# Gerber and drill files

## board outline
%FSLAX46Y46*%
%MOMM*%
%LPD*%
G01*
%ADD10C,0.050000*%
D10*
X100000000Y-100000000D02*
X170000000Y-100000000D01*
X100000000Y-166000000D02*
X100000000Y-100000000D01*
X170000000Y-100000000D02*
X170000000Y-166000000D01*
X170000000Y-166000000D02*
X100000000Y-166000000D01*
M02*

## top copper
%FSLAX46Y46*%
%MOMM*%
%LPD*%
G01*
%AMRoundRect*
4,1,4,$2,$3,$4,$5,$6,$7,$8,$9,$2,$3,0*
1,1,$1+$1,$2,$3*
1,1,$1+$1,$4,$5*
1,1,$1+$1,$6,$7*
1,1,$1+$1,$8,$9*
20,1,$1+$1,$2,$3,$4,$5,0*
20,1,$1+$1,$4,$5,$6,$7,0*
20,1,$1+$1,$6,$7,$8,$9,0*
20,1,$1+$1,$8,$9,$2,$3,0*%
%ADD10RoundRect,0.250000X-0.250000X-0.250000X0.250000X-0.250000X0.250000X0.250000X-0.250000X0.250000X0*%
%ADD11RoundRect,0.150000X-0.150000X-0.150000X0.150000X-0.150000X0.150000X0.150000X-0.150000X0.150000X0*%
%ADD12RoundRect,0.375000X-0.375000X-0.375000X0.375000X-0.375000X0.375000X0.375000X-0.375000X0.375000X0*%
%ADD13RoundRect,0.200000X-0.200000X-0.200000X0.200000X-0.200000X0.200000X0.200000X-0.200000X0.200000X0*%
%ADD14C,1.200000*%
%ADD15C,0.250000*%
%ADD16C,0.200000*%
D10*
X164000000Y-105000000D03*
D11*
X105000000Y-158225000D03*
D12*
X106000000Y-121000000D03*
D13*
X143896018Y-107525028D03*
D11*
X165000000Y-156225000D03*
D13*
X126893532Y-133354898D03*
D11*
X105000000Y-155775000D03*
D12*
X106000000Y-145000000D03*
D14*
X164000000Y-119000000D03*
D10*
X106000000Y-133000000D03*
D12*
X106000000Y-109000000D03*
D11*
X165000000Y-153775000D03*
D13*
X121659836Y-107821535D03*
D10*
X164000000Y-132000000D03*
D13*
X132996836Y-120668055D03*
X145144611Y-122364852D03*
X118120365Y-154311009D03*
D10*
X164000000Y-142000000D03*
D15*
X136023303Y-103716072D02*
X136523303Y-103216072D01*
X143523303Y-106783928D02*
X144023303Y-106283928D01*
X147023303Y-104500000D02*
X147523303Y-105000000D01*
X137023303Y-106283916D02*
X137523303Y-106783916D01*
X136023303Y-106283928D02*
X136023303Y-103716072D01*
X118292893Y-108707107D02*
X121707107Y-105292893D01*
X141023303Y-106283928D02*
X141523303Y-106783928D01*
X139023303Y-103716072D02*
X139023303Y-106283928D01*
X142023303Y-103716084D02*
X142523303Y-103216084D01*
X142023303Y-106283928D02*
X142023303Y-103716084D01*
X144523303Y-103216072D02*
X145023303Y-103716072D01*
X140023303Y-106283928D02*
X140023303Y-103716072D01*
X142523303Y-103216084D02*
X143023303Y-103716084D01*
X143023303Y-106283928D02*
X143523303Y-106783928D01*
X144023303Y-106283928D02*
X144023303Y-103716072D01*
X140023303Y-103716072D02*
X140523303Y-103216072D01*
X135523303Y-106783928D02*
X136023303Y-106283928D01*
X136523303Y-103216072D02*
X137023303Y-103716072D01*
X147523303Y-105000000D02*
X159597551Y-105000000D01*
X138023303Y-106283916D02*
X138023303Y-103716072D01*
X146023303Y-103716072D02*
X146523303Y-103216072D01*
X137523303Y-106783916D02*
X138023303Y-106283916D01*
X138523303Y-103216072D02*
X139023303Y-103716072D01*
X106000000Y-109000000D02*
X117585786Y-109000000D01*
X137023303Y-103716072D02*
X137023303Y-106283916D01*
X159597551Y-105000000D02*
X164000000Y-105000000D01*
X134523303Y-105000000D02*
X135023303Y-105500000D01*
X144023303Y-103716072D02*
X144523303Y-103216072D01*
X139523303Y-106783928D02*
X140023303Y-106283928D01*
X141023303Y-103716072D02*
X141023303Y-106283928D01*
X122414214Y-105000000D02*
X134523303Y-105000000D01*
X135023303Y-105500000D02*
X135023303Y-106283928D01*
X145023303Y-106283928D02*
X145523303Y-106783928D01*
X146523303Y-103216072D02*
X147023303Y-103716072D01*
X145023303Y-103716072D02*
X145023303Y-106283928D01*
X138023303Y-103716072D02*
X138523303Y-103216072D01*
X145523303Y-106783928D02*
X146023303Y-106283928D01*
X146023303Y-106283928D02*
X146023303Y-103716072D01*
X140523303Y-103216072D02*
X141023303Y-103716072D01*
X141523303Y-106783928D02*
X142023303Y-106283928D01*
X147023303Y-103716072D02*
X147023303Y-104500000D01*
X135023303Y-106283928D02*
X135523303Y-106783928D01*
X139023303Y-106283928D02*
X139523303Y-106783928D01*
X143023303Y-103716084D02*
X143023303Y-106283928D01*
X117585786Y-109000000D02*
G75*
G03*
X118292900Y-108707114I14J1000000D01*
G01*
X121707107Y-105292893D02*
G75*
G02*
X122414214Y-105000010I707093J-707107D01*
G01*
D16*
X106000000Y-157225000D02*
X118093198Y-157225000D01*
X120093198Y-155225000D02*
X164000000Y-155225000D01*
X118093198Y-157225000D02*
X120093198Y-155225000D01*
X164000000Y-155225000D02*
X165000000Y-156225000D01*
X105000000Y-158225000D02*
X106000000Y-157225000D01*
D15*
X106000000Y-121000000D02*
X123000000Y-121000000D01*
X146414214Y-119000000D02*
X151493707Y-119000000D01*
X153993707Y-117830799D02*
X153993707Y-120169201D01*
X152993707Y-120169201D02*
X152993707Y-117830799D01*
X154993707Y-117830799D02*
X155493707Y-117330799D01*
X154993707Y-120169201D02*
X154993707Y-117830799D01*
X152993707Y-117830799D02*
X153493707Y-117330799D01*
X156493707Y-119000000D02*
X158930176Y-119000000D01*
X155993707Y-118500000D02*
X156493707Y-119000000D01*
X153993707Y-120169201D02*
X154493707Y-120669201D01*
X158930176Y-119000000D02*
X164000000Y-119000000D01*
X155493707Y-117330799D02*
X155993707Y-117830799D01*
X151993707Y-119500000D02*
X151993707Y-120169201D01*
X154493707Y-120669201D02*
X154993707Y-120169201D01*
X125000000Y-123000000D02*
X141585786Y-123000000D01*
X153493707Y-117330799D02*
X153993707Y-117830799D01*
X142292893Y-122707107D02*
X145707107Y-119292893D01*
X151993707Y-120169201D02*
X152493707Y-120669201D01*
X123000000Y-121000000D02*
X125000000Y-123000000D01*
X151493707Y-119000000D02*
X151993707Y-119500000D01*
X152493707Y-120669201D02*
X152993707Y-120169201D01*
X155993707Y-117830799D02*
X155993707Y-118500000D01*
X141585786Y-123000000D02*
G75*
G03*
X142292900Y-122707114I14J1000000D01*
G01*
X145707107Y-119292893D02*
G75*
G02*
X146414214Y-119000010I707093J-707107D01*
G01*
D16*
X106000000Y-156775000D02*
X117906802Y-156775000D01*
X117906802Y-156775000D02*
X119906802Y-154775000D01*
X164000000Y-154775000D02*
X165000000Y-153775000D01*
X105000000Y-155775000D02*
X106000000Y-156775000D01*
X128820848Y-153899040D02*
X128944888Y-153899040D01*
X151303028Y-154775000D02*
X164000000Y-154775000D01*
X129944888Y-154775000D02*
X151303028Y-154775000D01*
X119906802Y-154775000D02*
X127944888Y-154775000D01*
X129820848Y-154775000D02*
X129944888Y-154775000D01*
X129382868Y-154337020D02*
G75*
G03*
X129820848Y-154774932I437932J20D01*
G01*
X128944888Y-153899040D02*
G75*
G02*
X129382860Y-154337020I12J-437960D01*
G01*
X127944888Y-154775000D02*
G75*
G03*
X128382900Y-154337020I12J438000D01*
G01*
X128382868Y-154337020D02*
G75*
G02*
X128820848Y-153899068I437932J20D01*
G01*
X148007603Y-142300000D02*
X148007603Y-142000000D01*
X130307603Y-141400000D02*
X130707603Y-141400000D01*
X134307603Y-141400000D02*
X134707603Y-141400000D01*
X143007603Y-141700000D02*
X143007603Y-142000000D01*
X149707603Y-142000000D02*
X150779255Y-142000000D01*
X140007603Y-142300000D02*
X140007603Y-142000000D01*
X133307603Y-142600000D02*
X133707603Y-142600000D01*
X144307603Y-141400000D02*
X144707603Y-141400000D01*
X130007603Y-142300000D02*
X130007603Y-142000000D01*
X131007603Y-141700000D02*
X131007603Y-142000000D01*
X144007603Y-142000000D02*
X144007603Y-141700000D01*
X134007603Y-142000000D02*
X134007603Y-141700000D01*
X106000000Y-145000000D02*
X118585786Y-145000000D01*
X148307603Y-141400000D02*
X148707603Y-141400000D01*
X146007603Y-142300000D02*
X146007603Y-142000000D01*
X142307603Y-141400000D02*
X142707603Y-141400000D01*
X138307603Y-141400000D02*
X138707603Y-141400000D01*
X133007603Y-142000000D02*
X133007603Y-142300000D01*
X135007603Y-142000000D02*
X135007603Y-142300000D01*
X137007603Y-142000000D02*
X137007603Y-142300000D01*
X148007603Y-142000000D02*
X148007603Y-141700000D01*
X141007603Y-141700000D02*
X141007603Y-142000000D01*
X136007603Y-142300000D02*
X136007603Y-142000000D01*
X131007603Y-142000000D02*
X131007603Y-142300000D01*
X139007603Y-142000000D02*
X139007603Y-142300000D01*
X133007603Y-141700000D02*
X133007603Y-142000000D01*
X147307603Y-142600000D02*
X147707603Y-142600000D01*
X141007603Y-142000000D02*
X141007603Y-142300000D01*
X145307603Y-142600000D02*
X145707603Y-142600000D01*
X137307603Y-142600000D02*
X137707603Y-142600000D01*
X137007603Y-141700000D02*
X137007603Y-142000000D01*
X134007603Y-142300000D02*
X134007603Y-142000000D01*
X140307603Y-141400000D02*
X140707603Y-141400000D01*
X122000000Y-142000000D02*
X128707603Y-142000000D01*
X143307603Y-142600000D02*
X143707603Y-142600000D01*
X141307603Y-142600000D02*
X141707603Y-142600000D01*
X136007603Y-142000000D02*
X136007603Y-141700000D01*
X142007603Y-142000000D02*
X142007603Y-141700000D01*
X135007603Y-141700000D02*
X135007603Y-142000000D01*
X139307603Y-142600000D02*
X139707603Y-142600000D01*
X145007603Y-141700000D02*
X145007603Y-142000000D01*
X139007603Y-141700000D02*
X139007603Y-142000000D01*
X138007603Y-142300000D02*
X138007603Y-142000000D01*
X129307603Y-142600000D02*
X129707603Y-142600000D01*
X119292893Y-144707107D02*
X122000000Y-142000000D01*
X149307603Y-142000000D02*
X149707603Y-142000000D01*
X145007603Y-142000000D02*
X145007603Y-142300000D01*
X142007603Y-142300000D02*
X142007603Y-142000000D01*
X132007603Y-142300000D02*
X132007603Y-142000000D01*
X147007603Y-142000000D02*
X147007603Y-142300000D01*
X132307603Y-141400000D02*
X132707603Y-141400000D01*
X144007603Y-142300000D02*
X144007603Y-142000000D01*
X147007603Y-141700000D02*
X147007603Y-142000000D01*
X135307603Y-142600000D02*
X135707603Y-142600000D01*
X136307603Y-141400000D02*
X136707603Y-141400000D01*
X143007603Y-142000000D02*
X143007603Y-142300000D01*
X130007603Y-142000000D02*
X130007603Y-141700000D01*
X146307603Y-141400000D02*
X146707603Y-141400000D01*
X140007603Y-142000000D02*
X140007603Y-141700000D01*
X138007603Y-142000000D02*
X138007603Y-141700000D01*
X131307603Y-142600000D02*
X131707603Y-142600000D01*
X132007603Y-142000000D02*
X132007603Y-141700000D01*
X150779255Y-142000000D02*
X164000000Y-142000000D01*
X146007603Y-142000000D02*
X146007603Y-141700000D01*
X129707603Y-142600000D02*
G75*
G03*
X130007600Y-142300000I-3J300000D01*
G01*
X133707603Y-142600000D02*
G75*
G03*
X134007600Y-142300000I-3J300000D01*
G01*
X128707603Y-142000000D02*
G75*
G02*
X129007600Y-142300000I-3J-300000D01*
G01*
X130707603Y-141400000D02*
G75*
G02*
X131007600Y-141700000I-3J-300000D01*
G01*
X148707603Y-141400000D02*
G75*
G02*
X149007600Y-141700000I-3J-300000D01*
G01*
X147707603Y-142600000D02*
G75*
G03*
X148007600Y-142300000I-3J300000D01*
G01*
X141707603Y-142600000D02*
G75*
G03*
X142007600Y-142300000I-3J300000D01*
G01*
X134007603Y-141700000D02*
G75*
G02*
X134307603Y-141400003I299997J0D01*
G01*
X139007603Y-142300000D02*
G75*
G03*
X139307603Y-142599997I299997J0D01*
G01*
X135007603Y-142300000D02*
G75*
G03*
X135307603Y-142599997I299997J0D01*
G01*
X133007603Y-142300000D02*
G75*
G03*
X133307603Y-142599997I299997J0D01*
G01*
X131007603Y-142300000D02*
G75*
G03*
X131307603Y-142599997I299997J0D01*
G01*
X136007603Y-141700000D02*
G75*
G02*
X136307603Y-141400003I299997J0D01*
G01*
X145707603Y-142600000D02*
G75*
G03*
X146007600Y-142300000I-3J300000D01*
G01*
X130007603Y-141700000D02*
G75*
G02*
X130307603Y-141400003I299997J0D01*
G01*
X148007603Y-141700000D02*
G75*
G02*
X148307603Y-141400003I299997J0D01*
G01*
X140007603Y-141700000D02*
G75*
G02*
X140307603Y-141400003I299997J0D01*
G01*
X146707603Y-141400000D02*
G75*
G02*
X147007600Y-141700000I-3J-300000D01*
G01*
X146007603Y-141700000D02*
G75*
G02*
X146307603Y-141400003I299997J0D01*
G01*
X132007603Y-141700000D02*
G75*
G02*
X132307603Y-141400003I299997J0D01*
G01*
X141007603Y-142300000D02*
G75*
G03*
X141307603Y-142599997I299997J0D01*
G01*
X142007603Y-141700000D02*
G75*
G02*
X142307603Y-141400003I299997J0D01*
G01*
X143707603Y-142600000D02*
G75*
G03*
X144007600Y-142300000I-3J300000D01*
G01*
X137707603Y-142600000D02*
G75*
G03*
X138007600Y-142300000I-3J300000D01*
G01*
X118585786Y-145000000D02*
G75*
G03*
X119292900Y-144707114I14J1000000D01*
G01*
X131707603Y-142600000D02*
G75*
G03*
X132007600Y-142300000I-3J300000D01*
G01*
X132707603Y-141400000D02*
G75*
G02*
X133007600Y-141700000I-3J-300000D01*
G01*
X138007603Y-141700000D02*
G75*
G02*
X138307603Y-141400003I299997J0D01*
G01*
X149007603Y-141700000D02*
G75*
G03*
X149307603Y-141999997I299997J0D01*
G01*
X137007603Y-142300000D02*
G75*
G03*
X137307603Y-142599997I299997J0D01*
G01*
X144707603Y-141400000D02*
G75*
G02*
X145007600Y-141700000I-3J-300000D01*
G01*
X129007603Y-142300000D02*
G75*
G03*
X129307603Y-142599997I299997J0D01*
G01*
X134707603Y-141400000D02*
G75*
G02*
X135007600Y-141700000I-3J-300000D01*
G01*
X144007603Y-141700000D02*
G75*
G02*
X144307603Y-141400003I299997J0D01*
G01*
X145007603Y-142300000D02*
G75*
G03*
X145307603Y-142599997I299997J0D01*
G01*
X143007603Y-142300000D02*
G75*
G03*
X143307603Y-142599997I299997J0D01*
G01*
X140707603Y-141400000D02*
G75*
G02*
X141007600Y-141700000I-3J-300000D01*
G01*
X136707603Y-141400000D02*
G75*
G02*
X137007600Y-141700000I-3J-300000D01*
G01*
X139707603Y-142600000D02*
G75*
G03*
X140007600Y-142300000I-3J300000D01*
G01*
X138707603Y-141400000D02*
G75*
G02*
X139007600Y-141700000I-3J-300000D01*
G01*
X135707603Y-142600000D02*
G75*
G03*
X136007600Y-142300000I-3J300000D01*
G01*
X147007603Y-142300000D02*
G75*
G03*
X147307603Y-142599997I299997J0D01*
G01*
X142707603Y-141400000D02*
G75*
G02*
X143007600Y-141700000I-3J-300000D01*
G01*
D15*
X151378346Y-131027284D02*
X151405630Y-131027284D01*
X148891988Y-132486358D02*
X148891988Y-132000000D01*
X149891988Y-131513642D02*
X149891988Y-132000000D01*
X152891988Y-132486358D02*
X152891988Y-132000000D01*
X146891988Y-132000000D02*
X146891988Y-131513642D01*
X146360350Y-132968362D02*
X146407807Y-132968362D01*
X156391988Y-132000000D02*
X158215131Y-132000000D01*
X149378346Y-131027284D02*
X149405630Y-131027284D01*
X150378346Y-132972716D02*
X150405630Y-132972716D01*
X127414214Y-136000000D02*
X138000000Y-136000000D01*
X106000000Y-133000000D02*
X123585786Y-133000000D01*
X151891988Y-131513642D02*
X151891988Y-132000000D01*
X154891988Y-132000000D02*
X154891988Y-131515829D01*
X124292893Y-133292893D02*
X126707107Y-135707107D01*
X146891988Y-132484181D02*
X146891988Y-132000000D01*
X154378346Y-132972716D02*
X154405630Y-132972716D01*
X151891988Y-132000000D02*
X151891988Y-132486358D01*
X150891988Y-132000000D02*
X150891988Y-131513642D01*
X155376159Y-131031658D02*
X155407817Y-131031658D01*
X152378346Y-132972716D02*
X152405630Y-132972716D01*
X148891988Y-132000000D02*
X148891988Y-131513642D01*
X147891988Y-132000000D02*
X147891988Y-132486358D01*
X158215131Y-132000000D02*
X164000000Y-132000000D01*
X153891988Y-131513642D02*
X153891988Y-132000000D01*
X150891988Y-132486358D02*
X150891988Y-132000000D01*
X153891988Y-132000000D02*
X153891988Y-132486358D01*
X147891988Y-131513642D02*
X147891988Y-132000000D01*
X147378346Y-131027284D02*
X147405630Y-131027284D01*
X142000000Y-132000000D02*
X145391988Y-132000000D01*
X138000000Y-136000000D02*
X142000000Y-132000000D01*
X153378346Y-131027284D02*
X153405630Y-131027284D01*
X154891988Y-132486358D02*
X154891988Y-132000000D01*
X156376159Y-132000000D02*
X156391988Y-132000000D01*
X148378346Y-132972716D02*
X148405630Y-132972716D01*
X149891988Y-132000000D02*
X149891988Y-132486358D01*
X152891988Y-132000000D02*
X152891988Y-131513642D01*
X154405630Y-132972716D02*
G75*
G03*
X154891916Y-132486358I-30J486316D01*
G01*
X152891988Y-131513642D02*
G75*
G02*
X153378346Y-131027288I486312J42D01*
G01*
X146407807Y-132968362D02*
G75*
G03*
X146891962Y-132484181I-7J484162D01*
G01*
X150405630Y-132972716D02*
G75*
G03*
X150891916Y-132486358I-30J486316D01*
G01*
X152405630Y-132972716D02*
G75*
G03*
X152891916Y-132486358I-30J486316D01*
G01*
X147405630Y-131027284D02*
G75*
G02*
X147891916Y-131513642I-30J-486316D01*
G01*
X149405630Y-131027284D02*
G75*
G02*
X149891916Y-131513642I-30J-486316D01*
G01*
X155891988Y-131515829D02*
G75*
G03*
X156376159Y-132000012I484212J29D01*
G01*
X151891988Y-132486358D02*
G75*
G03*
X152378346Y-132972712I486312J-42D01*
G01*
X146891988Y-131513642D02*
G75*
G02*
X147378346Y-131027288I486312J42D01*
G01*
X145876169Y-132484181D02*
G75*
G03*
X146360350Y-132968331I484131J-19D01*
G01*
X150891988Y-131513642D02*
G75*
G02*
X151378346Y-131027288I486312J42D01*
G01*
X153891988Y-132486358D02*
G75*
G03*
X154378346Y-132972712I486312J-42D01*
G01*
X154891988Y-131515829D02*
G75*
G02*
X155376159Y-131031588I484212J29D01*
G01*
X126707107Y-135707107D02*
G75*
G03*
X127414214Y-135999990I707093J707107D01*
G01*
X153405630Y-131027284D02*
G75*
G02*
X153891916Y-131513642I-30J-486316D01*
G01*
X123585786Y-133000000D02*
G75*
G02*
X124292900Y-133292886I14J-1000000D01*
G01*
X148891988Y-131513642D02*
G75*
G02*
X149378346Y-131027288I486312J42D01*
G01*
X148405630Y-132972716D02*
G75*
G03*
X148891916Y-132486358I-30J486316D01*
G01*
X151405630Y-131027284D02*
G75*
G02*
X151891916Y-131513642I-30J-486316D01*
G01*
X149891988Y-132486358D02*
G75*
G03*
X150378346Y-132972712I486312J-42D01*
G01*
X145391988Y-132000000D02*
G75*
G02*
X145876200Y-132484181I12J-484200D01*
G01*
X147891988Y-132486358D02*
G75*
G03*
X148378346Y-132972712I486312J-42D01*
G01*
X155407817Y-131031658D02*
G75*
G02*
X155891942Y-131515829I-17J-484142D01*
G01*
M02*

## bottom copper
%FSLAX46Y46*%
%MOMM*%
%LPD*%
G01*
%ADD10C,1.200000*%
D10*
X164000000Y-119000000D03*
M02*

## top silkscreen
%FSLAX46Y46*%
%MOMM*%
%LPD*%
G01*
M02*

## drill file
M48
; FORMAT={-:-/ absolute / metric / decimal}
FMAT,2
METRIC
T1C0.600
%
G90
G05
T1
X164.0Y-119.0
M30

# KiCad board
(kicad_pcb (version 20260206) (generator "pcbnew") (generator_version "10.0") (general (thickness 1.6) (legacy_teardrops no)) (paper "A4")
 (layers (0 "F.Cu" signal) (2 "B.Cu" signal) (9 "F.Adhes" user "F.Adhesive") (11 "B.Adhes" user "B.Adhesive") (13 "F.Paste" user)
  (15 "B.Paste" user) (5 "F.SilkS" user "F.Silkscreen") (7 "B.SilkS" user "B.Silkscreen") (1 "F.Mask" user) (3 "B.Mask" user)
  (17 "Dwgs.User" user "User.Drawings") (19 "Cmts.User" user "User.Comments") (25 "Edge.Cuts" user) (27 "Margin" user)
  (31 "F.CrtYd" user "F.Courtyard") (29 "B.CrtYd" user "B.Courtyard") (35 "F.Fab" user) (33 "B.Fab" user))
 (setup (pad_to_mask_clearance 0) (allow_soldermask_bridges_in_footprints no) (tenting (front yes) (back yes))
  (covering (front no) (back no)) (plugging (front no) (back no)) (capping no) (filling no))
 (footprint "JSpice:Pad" (layer "F.Cu") (at 164 105)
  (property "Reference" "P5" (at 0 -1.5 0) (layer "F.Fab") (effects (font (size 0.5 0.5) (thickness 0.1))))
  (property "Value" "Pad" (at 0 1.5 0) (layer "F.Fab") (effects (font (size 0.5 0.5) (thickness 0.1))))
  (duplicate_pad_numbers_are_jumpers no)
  (pad "1" smd roundrect (at 0 0) (size 1 1) (layers "F.Cu" "F.Mask") (roundrect_rratio 0.25) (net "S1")))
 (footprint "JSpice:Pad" (layer "F.Cu") (at 105 158.225)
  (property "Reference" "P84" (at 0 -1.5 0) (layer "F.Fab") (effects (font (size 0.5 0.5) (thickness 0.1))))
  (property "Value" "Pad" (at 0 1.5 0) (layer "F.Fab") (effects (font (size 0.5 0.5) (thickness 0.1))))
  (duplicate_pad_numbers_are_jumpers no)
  (pad "1" smd roundrect (at 0 0) (size 0.6 0.6) (layers "F.Cu" "F.Mask") (roundrect_rratio 0.25) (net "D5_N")))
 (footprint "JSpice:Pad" (layer "F.Cu") (at 106 121)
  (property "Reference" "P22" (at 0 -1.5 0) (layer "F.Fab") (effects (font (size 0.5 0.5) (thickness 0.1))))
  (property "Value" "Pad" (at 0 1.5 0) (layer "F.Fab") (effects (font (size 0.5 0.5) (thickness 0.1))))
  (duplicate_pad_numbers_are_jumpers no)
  (pad "1" smd roundrect (at 0 0) (size 1.5 1.5) (layers "F.Cu" "F.Mask") (roundrect_rratio 0.25) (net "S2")))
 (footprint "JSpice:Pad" (layer "F.Cu") (at 143.896018 107.525028)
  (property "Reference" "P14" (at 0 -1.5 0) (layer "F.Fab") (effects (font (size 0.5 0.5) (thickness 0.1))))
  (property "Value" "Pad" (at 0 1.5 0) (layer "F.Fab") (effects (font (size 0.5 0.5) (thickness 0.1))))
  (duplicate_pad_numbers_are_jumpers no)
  (pad "1" smd roundrect (at 0 0) (size 0.8 0.8) (layers "F.Cu" "F.Mask") (roundrect_rratio 0.25) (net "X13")))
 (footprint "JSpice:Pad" (layer "F.Cu") (at 165 156.225)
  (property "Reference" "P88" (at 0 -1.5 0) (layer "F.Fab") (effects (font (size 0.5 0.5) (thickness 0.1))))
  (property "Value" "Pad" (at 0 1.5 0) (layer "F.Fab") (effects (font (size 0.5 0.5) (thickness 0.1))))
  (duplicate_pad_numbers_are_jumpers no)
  (pad "1" smd roundrect (at 0 0) (size 0.6 0.6) (layers "F.Cu" "F.Mask") (roundrect_rratio 0.25) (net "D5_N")))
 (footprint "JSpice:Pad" (layer "F.Cu") (at 126.893532 133.354898)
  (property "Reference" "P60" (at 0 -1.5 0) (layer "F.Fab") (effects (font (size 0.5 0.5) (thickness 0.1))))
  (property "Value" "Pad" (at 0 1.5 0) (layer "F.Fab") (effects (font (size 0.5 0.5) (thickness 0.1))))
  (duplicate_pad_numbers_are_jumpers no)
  (pad "1" smd roundrect (at 0 0) (size 0.8 0.8) (layers "F.Cu" "F.Mask") (roundrect_rratio 0.25) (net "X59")))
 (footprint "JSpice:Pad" (layer "F.Cu") (at 105 155.775)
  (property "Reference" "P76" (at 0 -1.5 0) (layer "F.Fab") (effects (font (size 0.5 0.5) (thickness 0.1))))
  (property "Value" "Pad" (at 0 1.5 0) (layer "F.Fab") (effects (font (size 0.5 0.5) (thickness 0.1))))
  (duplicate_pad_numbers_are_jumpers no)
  (pad "1" smd roundrect (at 0 0) (size 0.6 0.6) (layers "F.Cu" "F.Mask") (roundrect_rratio 0.25) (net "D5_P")))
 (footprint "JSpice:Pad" (layer "F.Cu") (at 106 145)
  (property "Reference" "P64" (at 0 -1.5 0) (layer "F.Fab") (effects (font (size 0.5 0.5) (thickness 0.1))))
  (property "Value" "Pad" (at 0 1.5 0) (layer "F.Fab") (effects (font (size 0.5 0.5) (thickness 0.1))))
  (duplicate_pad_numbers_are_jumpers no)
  (pad "1" smd roundrect (at 0 0) (size 1.5 1.5) (layers "F.Cu" "F.Mask") (roundrect_rratio 0.25) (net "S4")))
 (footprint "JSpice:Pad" (layer "F.Cu") (at 164 119)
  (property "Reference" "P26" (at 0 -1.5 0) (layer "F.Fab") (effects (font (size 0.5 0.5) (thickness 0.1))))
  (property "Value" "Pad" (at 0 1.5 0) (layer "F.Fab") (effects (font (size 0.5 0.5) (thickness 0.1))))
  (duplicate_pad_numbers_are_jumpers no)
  (pad "1" thru_hole circle (at 0 0) (size 1.2 1.2) (drill 0.6) (layers "*.Cu" "*.Mask") (remove_unused_layers no) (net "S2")))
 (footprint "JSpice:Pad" (layer "F.Cu") (at 106 133)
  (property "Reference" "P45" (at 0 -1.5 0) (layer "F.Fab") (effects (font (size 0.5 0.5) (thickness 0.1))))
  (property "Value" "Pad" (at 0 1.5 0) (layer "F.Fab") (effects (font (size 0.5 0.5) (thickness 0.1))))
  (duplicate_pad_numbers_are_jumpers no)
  (pad "1" smd roundrect (at 0 0) (size 1 1) (layers "F.Cu" "F.Mask") (roundrect_rratio 0.25) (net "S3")))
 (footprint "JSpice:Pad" (layer "F.Cu") (at 106 109)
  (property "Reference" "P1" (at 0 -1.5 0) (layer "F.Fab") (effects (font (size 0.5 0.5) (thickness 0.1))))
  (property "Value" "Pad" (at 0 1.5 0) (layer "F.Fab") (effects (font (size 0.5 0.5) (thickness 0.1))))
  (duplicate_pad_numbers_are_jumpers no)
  (pad "1" smd roundrect (at 0 0) (size 1.5 1.5) (layers "F.Cu" "F.Mask") (roundrect_rratio 0.25) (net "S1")))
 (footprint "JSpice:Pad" (layer "F.Cu") (at 165 153.775)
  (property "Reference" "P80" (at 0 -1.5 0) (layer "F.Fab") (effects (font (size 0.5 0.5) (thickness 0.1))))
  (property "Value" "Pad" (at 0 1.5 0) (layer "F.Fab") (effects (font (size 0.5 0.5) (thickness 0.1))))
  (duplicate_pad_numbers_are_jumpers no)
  (pad "1" smd roundrect (at 0 0) (size 0.6 0.6) (layers "F.Cu" "F.Mask") (roundrect_rratio 0.25) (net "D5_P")))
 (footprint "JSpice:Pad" (layer "F.Cu") (at 121.659836 107.821535)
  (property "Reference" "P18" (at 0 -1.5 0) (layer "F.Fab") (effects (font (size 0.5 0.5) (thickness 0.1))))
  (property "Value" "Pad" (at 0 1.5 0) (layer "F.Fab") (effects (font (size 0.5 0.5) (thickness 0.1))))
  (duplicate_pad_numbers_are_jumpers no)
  (pad "1" smd roundrect (at 0 0) (size 0.8 0.8) (layers "F.Cu" "F.Mask") (roundrect_rratio 0.25) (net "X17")))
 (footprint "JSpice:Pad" (layer "F.Cu") (at 164 132)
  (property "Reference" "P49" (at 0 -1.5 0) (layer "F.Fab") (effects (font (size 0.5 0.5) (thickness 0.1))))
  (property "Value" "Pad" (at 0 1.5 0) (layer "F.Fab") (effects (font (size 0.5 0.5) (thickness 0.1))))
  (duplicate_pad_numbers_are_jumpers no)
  (pad "1" smd roundrect (at 0 0) (size 1 1) (layers "F.Cu" "F.Mask") (roundrect_rratio 0.25) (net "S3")))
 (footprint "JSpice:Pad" (layer "F.Cu") (at 132.996836 120.668055)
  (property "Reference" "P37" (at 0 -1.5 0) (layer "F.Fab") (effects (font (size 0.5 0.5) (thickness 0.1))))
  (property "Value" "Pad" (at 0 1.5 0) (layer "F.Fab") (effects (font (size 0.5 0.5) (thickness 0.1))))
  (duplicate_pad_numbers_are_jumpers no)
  (pad "1" smd roundrect (at 0 0) (size 0.8 0.8) (layers "F.Cu" "F.Mask") (roundrect_rratio 0.25) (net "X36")))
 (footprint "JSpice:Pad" (layer "F.Cu") (at 145.144611 122.364852)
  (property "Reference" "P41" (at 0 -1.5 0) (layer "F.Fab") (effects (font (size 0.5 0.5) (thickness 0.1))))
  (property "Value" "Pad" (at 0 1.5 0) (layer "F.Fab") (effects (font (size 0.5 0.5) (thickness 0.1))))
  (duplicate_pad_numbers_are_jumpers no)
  (pad "1" smd roundrect (at 0 0) (size 0.8 0.8) (layers "F.Cu" "F.Mask") (roundrect_rratio 0.25) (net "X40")))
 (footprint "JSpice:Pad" (layer "F.Cu") (at 118.120365 154.311009)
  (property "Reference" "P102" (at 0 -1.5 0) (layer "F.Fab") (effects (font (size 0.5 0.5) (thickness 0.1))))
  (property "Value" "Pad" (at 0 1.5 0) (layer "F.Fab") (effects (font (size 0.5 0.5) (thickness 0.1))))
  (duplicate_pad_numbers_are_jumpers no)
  (pad "1" smd roundrect (at 0 0) (size 0.8 0.8) (layers "F.Cu" "F.Mask") (roundrect_rratio 0.25) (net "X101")))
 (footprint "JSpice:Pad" (layer "F.Cu") (at 164 142)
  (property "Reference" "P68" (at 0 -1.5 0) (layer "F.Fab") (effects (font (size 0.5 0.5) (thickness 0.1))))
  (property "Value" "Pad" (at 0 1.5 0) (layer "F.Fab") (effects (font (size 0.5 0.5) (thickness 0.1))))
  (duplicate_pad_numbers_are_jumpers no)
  (pad "1" smd roundrect (at 0 0) (size 1 1) (layers "F.Cu" "F.Mask") (roundrect_rratio 0.25) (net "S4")))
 (gr_line (start 100 100) (end 170 100) (stroke (width 0.05) (type default)) (layer "Edge.Cuts"))
 (gr_line (start 100 166) (end 100 100) (stroke (width 0.05) (type default)) (layer "Edge.Cuts"))
 (gr_line (start 170 100) (end 170 166) (stroke (width 0.05) (type default)) (layer "Edge.Cuts"))
 (gr_line (start 170 166) (end 100 166) (stroke (width 0.05) (type default)) (layer "Edge.Cuts"))
 (segment (start 136.023303 103.716072) (end 136.523303 103.216072) (width 0.25) (layer "F.Cu") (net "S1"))
 (segment (start 143.523303 106.783928) (end 144.023303 106.283928) (width 0.25) (layer "F.Cu") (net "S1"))
 (segment (start 147.023303 104.5) (end 147.523303 105) (width 0.25) (layer "F.Cu") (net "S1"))
 (segment (start 137.023303 106.283916) (end 137.523303 106.783916) (width 0.25) (layer "F.Cu") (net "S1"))
 (segment (start 136.023303 106.283928) (end 136.023303 103.716072) (width 0.25) (layer "F.Cu") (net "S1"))
 (segment (start 118.292893 108.707107) (end 121.707107 105.292893) (width 0.25) (layer "F.Cu") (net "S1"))
 (segment (start 141.023303 106.283928) (end 141.523303 106.783928) (width 0.25) (layer "F.Cu") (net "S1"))
 (segment (start 139.023303 103.716072) (end 139.023303 106.283928) (width 0.25) (layer "F.Cu") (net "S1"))
 (segment (start 142.023303 103.716084) (end 142.523303 103.216084) (width 0.25) (layer "F.Cu") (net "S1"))
 (segment (start 142.023303 106.283928) (end 142.023303 103.716084) (width 0.25) (layer "F.Cu") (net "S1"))
 (segment (start 144.523303 103.216072) (end 145.023303 103.716072) (width 0.25) (layer "F.Cu") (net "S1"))
 (segment (start 140.023303 106.283928) (end 140.023303 103.716072) (width 0.25) (layer "F.Cu") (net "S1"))
 (segment (start 142.523303 103.216084) (end 143.023303 103.716084) (width 0.25) (layer "F.Cu") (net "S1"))
 (segment (start 143.023303 106.283928) (end 143.523303 106.783928) (width 0.25) (layer "F.Cu") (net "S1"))
 (segment (start 144.023303 106.283928) (end 144.023303 103.716072) (width 0.25) (layer "F.Cu") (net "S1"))
 (segment (start 140.023303 103.716072) (end 140.523303 103.216072) (width 0.25) (layer "F.Cu") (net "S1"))
 (segment (start 135.523303 106.783928) (end 136.023303 106.283928) (width 0.25) (layer "F.Cu") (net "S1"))
 (segment (start 136.523303 103.216072) (end 137.023303 103.716072) (width 0.25) (layer "F.Cu") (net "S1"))
 (segment (start 147.523303 105) (end 159.597551 105) (width 0.25) (layer "F.Cu") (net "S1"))
 (segment (start 138.023303 106.283916) (end 138.023303 103.716072) (width 0.25) (layer "F.Cu") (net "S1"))
 (segment (start 146.023303 103.716072) (end 146.523303 103.216072) (width 0.25) (layer "F.Cu") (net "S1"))
 (segment (start 137.523303 106.783916) (end 138.023303 106.283916) (width 0.25) (layer "F.Cu") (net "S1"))
 (segment (start 138.523303 103.216072) (end 139.023303 103.716072) (width 0.25) (layer "F.Cu") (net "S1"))
 (segment (start 106 109) (end 117.585786 109) (width 0.25) (layer "F.Cu") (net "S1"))
 (segment (start 137.023303 103.716072) (end 137.023303 106.283916) (width 0.25) (layer "F.Cu") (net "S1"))
 (segment (start 159.597551 105) (end 164 105) (width 0.25) (layer "F.Cu") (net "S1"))
 (segment (start 134.523303 105) (end 135.023303 105.5) (width 0.25) (layer "F.Cu") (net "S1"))
 (segment (start 144.023303 103.716072) (end 144.523303 103.216072) (width 0.25) (layer "F.Cu") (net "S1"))
 (segment (start 139.523303 106.783928) (end 140.023303 106.283928) (width 0.25) (layer "F.Cu") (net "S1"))
 (segment (start 141.023303 103.716072) (end 141.023303 106.283928) (width 0.25) (layer "F.Cu") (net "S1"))
 (segment (start 122.414214 105) (end 134.523303 105) (width 0.25) (layer "F.Cu") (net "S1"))
 (segment (start 135.023303 105.5) (end 135.023303 106.283928) (width 0.25) (layer "F.Cu") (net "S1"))
 (segment (start 145.023303 106.283928) (end 145.523303 106.783928) (width 0.25) (layer "F.Cu") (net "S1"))
 (segment (start 146.523303 103.216072) (end 147.023303 103.716072) (width 0.25) (layer "F.Cu") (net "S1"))
 (segment (start 145.023303 103.716072) (end 145.023303 106.283928) (width 0.25) (layer "F.Cu") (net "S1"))
 (segment (start 138.023303 103.716072) (end 138.523303 103.216072) (width 0.25) (layer "F.Cu") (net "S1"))
 (segment (start 145.523303 106.783928) (end 146.023303 106.283928) (width 0.25) (layer "F.Cu") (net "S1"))
 (segment (start 146.023303 106.283928) (end 146.023303 103.716072) (width 0.25) (layer "F.Cu") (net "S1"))
 (segment (start 140.523303 103.216072) (end 141.023303 103.716072) (width 0.25) (layer "F.Cu") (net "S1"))
 (segment (start 141.523303 106.783928) (end 142.023303 106.283928) (width 0.25) (layer "F.Cu") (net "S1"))
 (segment (start 147.023303 103.716072) (end 147.023303 104.5) (width 0.25) (layer "F.Cu") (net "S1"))
 (segment (start 135.023303 106.283928) (end 135.523303 106.783928) (width 0.25) (layer "F.Cu") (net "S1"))
 (segment (start 139.023303 106.283928) (end 139.523303 106.783928) (width 0.25) (layer "F.Cu") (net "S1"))
 (segment (start 143.023303 103.716084) (end 143.023303 106.283928) (width 0.25) (layer "F.Cu") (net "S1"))
 (arc (start 117.585786 109) (mid 117.96847 108.92388) (end 118.292893 108.707107) (width 0.25) (layer "F.Cu") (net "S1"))
 (arc (start 121.707107 105.292893) (mid 122.03153 105.07612) (end 122.414214 105) (width 0.25) (layer "F.Cu") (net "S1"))
 (segment (start 106 157.225) (end 118.093198 157.225) (width 0.2) (layer "F.Cu") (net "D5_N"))
 (segment (start 120.093198 155.225) (end 164 155.225) (width 0.2) (layer "F.Cu") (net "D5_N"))
 (segment (start 118.093198 157.225) (end 120.093198 155.225) (width 0.2) (layer "F.Cu") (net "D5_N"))
 (segment (start 164 155.225) (end 165 156.225) (width 0.2) (layer "F.Cu") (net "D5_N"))
 (segment (start 105 158.225) (end 106 157.225) (width 0.2) (layer "F.Cu") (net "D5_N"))
 (segment (start 106 121) (end 123 121) (width 0.25) (layer "F.Cu") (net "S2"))
 (segment (start 146.414214 119) (end 151.493707 119) (width 0.25) (layer "F.Cu") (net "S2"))
 (segment (start 153.993707 117.830799) (end 153.993707 120.169201) (width 0.25) (layer "F.Cu") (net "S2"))
 (segment (start 152.993707 120.169201) (end 152.993707 117.830799) (width 0.25) (layer "F.Cu") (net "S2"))
 (segment (start 154.993707 117.830799) (end 155.493707 117.330799) (width 0.25) (layer "F.Cu") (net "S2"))
 (segment (start 154.993707 120.169201) (end 154.993707 117.830799) (width 0.25) (layer "F.Cu") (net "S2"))
 (segment (start 152.993707 117.830799) (end 153.493707 117.330799) (width 0.25) (layer "F.Cu") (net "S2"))
 (segment (start 156.493707 119) (end 158.930176 119) (width 0.25) (layer "F.Cu") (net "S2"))
 (segment (start 155.993707 118.5) (end 156.493707 119) (width 0.25) (layer "F.Cu") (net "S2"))
 (segment (start 153.993707 120.169201) (end 154.493707 120.669201) (width 0.25) (layer "F.Cu") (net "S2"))
 (segment (start 158.930176 119) (end 164 119) (width 0.25) (layer "F.Cu") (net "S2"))
 (segment (start 155.493707 117.330799) (end 155.993707 117.830799) (width 0.25) (layer "F.Cu") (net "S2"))
 (segment (start 151.993707 119.5) (end 151.993707 120.169201) (width 0.25) (layer "F.Cu") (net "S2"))
 (segment (start 154.493707 120.669201) (end 154.993707 120.169201) (width 0.25) (layer "F.Cu") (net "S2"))
 (segment (start 125 123) (end 141.585786 123) (width 0.25) (layer "F.Cu") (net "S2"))
 (segment (start 153.493707 117.330799) (end 153.993707 117.830799) (width 0.25) (layer "F.Cu") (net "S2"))
 (segment (start 142.292893 122.707107) (end 145.707107 119.292893) (width 0.25) (layer "F.Cu") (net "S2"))
 (segment (start 151.993707 120.169201) (end 152.493707 120.669201) (width 0.25) (layer "F.Cu") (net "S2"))
 (segment (start 123 121) (end 125 123) (width 0.25) (layer "F.Cu") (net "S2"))
 (segment (start 151.493707 119) (end 151.993707 119.5) (width 0.25) (layer "F.Cu") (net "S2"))
 (segment (start 152.493707 120.669201) (end 152.993707 120.169201) (width 0.25) (layer "F.Cu") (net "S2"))
 (segment (start 155.993707 117.830799) (end 155.993707 118.5) (width 0.25) (layer "F.Cu") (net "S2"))
 (arc (start 141.585786 123) (mid 141.96847 122.92388) (end 142.292893 122.707107) (width 0.25) (layer "F.Cu") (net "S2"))
 (arc (start 145.707107 119.292893) (mid 146.03153 119.07612) (end 146.414214 119) (width 0.25) (layer "F.Cu") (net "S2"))
 (segment (start 106 156.775) (end 117.906802 156.775) (width 0.2) (layer "F.Cu") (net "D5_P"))
 (segment (start 117.906802 156.775) (end 119.906802 154.775) (width 0.2) (layer "F.Cu") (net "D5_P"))
 (segment (start 164 154.775) (end 165 153.775) (width 0.2) (layer "F.Cu") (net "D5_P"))
 (segment (start 105 155.775) (end 106 156.775) (width 0.2) (layer "F.Cu") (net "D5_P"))
 (segment (start 128.820848 153.89904) (end 128.944888 153.89904) (width 0.2) (layer "F.Cu") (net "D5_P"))
 (segment (start 151.303028 154.775) (end 164 154.775) (width 0.2) (layer "F.Cu") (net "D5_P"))
 (segment (start 129.944888 154.775) (end 151.303028 154.775) (width 0.2) (layer "F.Cu") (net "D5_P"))
 (segment (start 119.906802 154.775) (end 127.944888 154.775) (width 0.2) (layer "F.Cu") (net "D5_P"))
 (segment (start 129.820848 154.775) (end 129.944888 154.775) (width 0.2) (layer "F.Cu") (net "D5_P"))
 (arc (start 129.382868 154.33702) (mid 129.511149 154.646719) (end 129.820848 154.775) (width 0.2) (layer "F.Cu") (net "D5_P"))
 (arc (start 128.944888 153.89904) (mid 129.254587 154.027321) (end 129.382868 154.33702) (width 0.2) (layer "F.Cu") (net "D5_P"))
 (arc (start 127.944888 154.775) (mid 128.254587 154.646719) (end 128.382868 154.33702) (width 0.2) (layer "F.Cu") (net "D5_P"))
 (arc (start 128.382868 154.33702) (mid 128.511149 154.027321) (end 128.820848 153.89904) (width 0.2) (layer "F.Cu") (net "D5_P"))
 (segment (start 148.007603 142.3) (end 148.007603 142) (width 0.2) (layer "F.Cu") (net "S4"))
 (segment (start 130.307603 141.4) (end 130.707603 141.4) (width 0.2) (layer "F.Cu") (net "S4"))
 (segment (start 134.307603 141.4) (end 134.707603 141.4) (width 0.2) (layer "F.Cu") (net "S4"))
 (segment (start 143.007603 141.7) (end 143.007603 142) (width 0.2) (layer "F.Cu") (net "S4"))
 (segment (start 149.707603 142) (end 150.779255 142) (width 0.2) (layer "F.Cu") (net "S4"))
 (segment (start 140.007603 142.3) (end 140.007603 142) (width 0.2) (layer "F.Cu") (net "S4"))
 (segment (start 133.307603 142.6) (end 133.707603 142.6) (width 0.2) (layer "F.Cu") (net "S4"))
 (segment (start 144.307603 141.4) (end 144.707603 141.4) (width 0.2) (layer "F.Cu") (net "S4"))
 (segment (start 130.007603 142.3) (end 130.007603 142) (width 0.2) (layer "F.Cu") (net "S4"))
 (segment (start 131.007603 141.7) (end 131.007603 142) (width 0.2) (layer "F.Cu") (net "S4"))
 (segment (start 144.007603 142) (end 144.007603 141.7) (width 0.2) (layer "F.Cu") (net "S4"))
 (segment (start 134.007603 142) (end 134.007603 141.7) (width 0.2) (layer "F.Cu") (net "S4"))
 (segment (start 106 145) (end 118.585786 145) (width 0.2) (layer "F.Cu") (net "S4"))
 (segment (start 148.307603 141.4) (end 148.707603 141.4) (width 0.2) (layer "F.Cu") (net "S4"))
 (segment (start 146.007603 142.3) (end 146.007603 142) (width 0.2) (layer "F.Cu") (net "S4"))
 (segment (start 142.307603 141.4) (end 142.707603 141.4) (width 0.2) (layer "F.Cu") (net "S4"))
 (segment (start 138.307603 141.4) (end 138.707603 141.4) (width 0.2) (layer "F.Cu") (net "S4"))
 (segment (start 133.007603 142) (end 133.007603 142.3) (width 0.2) (layer "F.Cu") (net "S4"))
 (segment (start 135.007603 142) (end 135.007603 142.3) (width 0.2) (layer "F.Cu") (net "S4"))
 (segment (start 137.007603 142) (end 137.007603 142.3) (width 0.2) (layer "F.Cu") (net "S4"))
 (segment (start 148.007603 142) (end 148.007603 141.7) (width 0.2) (layer "F.Cu") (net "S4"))
 (segment (start 141.007603 141.7) (end 141.007603 142) (width 0.2) (layer "F.Cu") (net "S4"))
 (segment (start 136.007603 142.3) (end 136.007603 142) (width 0.2) (layer "F.Cu") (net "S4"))
 (segment (start 131.007603 142) (end 131.007603 142.3) (width 0.2) (layer "F.Cu") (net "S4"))
 (segment (start 139.007603 142) (end 139.007603 142.3) (width 0.2) (layer "F.Cu") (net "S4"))
 (segment (start 133.007603 141.7) (end 133.007603 142) (width 0.2) (layer "F.Cu") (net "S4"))
 (segment (start 147.307603 142.6) (end 147.707603 142.6) (width 0.2) (layer "F.Cu") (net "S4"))
 (segment (start 141.007603 142) (end 141.007603 142.3) (width 0.2) (layer "F.Cu") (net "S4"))
 (segment (start 145.307603 142.6) (end 145.707603 142.6) (width 0.2) (layer "F.Cu") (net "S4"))
 (segment (start 137.307603 142.6) (end 137.707603 142.6) (width 0.2) (layer "F.Cu") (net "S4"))
 (segment (start 137.007603 141.7) (end 137.007603 142) (width 0.2) (layer "F.Cu") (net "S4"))
 (segment (start 134.007603 142.3) (end 134.007603 142) (width 0.2) (layer "F.Cu") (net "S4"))
 (segment (start 140.307603 141.4) (end 140.707603 141.4) (width 0.2) (layer "F.Cu") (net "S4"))
 (segment (start 122 142) (end 128.707603 142) (width 0.2) (layer "F.Cu") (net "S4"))
 (segment (start 143.307603 142.6) (end 143.707603 142.6) (width 0.2) (layer "F.Cu") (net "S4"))
 (segment (start 141.307603 142.6) (end 141.707603 142.6) (width 0.2) (layer "F.Cu") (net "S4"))
 (segment (start 136.007603 142) (end 136.007603 141.7) (width 0.2) (layer "F.Cu") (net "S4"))
 (segment (start 142.007603 142) (end 142.007603 141.7) (width 0.2) (layer "F.Cu") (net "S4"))
 (segment (start 135.007603 141.7) (end 135.007603 142) (width 0.2) (layer "F.Cu") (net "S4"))
 (segment (start 139.307603 142.6) (end 139.707603 142.6) (width 0.2) (layer "F.Cu") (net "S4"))
 (segment (start 145.007603 141.7) (end 145.007603 142) (width 0.2) (layer "F.Cu") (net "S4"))
 (segment (start 139.007603 141.7) (end 139.007603 142) (width 0.2) (layer "F.Cu") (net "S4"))
 (segment (start 138.007603 142.3) (end 138.007603 142) (width 0.2) (layer "F.Cu") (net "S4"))
 (segment (start 129.307603 142.6) (end 129.707603 142.6) (width 0.2) (layer "F.Cu") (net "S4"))
 (segment (start 119.292893 144.707107) (end 122 142) (width 0.2) (layer "F.Cu") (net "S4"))
 (segment (start 149.307603 142) (end 149.707603 142) (width 0.2) (layer "F.Cu") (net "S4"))
 (segment (start 145.007603 142) (end 145.007603 142.3) (width 0.2) (layer "F.Cu") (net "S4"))
 (segment (start 142.007603 142.3) (end 142.007603 142) (width 0.2) (layer "F.Cu") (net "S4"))
 (segment (start 132.007603 142.3) (end 132.007603 142) (width 0.2) (layer "F.Cu") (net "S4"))
 (segment (start 147.007603 142) (end 147.007603 142.3) (width 0.2) (layer "F.Cu") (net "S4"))
 (segment (start 132.307603 141.4) (end 132.707603 141.4) (width 0.2) (layer "F.Cu") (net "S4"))
 (segment (start 144.007603 142.3) (end 144.007603 142) (width 0.2) (layer "F.Cu") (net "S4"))
 (segment (start 147.007603 141.7) (end 147.007603 142) (width 0.2) (layer "F.Cu") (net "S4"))
 (segment (start 135.307603 142.6) (end 135.707603 142.6) (width 0.2) (layer "F.Cu") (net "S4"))
 (segment (start 136.307603 141.4) (end 136.707603 141.4) (width 0.2) (layer "F.Cu") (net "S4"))
 (segment (start 143.007603 142) (end 143.007603 142.3) (width 0.2) (layer "F.Cu") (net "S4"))
 (segment (start 130.007603 142) (end 130.007603 141.7) (width 0.2) (layer "F.Cu") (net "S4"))
 (segment (start 146.307603 141.4) (end 146.707603 141.4) (width 0.2) (layer "F.Cu") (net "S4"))
 (segment (start 140.007603 142) (end 140.007603 141.7) (width 0.2) (layer "F.Cu") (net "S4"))
 (segment (start 138.007603 142) (end 138.007603 141.7) (width 0.2) (layer "F.Cu") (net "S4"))
 (segment (start 131.307603 142.6) (end 131.707603 142.6) (width 0.2) (layer "F.Cu") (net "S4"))
 (segment (start 132.007603 142) (end 132.007603 141.7) (width 0.2) (layer "F.Cu") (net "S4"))
 (segment (start 150.779255 142) (end 164 142) (width 0.2) (layer "F.Cu") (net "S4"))
 (segment (start 146.007603 142) (end 146.007603 141.7) (width 0.2) (layer "F.Cu") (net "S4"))
 (arc (start 129.707603 142.6) (mid 129.919735 142.512132) (end 130.007603 142.3) (width 0.2) (layer "F.Cu") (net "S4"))
 (arc (start 133.707603 142.6) (mid 133.919735 142.512132) (end 134.007603 142.3) (width 0.2) (layer "F.Cu") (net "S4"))
 (arc (start 128.707603 142) (mid 128.919735 142.087868) (end 129.007603 142.3) (width 0.2) (layer "F.Cu") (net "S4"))
 (arc (start 130.707603 141.4) (mid 130.919735 141.487868) (end 131.007603 141.7) (width 0.2) (layer "F.Cu") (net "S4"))
 (arc (start 148.707603 141.4) (mid 148.919735 141.487868) (end 149.007603 141.7) (width 0.2) (layer "F.Cu") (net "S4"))
 (arc (start 147.707603 142.6) (mid 147.919735 142.512132) (end 148.007603 142.3) (width 0.2) (layer "F.Cu") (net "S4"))
 (arc (start 141.707603 142.6) (mid 141.919735 142.512132) (end 142.007603 142.3) (width 0.2) (layer "F.Cu") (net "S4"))
 (arc (start 134.007603 141.7) (mid 134.095471 141.487868) (end 134.307603 141.4) (width 0.2) (layer "F.Cu") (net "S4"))
 (arc (start 139.007603 142.3) (mid 139.095471 142.512132) (end 139.307603 142.6) (width 0.2) (layer "F.Cu") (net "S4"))
 (arc (start 135.007603 142.3) (mid 135.095471 142.512132) (end 135.307603 142.6) (width 0.2) (layer "F.Cu") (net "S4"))
 (arc (start 133.007603 142.3) (mid 133.095471 142.512132) (end 133.307603 142.6) (width 0.2) (layer "F.Cu") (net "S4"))
 (arc (start 131.007603 142.3) (mid 131.095471 142.512132) (end 131.307603 142.6) (width 0.2) (layer "F.Cu") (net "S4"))
 (arc (start 136.007603 141.7) (mid 136.095471 141.487868) (end 136.307603 141.4) (width 0.2) (layer "F.Cu") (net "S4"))
 (arc (start 145.707603 142.6) (mid 145.919735 142.512132) (end 146.007603 142.3) (width 0.2) (layer "F.Cu") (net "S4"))
 (arc (start 130.007603 141.7) (mid 130.095471 141.487868) (end 130.307603 141.4) (width 0.2) (layer "F.Cu") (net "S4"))
 (arc (start 148.007603 141.7) (mid 148.095471 141.487868) (end 148.307603 141.4) (width 0.2) (layer "F.Cu") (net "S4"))
 (arc (start 140.007603 141.7) (mid 140.095471 141.487868) (end 140.307603 141.4) (width 0.2) (layer "F.Cu") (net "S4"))
 (arc (start 146.707603 141.4) (mid 146.919735 141.487868) (end 147.007603 141.7) (width 0.2) (layer "F.Cu") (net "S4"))
 (arc (start 146.007603 141.7) (mid 146.095471 141.487868) (end 146.307603 141.4) (width 0.2) (layer "F.Cu") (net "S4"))
 (arc (start 132.007603 141.7) (mid 132.095471 141.487868) (end 132.307603 141.4) (width 0.2) (layer "F.Cu") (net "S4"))
 (arc (start 141.007603 142.3) (mid 141.095471 142.512132) (end 141.307603 142.6) (width 0.2) (layer "F.Cu") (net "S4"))
 (arc (start 142.007603 141.7) (mid 142.095471 141.487868) (end 142.307603 141.4) (width 0.2) (layer "F.Cu") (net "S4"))
 (arc (start 143.707603 142.6) (mid 143.919735 142.512132) (end 144.007603 142.3) (width 0.2) (layer "F.Cu") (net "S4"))
 (arc (start 137.707603 142.6) (mid 137.919735 142.512132) (end 138.007603 142.3) (width 0.2) (layer "F.Cu") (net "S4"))
 (arc (start 118.585786 145) (mid 118.96847 144.92388) (end 119.292893 144.707107) (width 0.2) (layer "F.Cu") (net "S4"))
 (arc (start 131.707603 142.6) (mid 131.919735 142.512132) (end 132.007603 142.3) (width 0.2) (layer "F.Cu") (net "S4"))
 (arc (start 132.707603 141.4) (mid 132.919735 141.487868) (end 133.007603 141.7) (width 0.2) (layer "F.Cu") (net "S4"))
 (arc (start 138.007603 141.7) (mid 138.095471 141.487868) (end 138.307603 141.4) (width 0.2) (layer "F.Cu") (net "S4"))
 (arc (start 149.007603 141.7) (mid 149.095471 141.912132) (end 149.307603 142) (width 0.2) (layer "F.Cu") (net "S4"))
 (arc (start 137.007603 142.3) (mid 137.095471 142.512132) (end 137.307603 142.6) (width 0.2) (layer "F.Cu") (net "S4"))
 (arc (start 144.707603 141.4) (mid 144.919735 141.487868) (end 145.007603 141.7) (width 0.2) (layer "F.Cu") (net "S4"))
 (arc (start 129.007603 142.3) (mid 129.095471 142.512132) (end 129.307603 142.6) (width 0.2) (layer "F.Cu") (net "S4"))
 (arc (start 134.707603 141.4) (mid 134.919735 141.487868) (end 135.007603 141.7) (width 0.2) (layer "F.Cu") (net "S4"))
 (arc (start 144.007603 141.7) (mid 144.095471 141.487868) (end 144.307603 141.4) (width 0.2) (layer "F.Cu") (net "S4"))
 (arc (start 145.007603 142.3) (mid 145.095471 142.512132) (end 145.307603 142.6) (width 0.2) (layer "F.Cu") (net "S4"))
 (arc (start 143.007603 142.3) (mid 143.095471 142.512132) (end 143.307603 142.6) (width 0.2) (layer "F.Cu") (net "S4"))
 (arc (start 140.707603 141.4) (mid 140.919735 141.487868) (end 141.007603 141.7) (width 0.2) (layer "F.Cu") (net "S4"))
 (arc (start 136.707603 141.4) (mid 136.919735 141.487868) (end 137.007603 141.7) (width 0.2) (layer "F.Cu") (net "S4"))
 (arc (start 139.707603 142.6) (mid 139.919735 142.512132) (end 140.007603 142.3) (width 0.2) (layer "F.Cu") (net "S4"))
 (arc (start 138.707603 141.4) (mid 138.919735 141.487868) (end 139.007603 141.7) (width 0.2) (layer "F.Cu") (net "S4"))
 (arc (start 135.707603 142.6) (mid 135.919735 142.512132) (end 136.007603 142.3) (width 0.2) (layer "F.Cu") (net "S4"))
 (arc (start 147.007603 142.3) (mid 147.095471 142.512132) (end 147.307603 142.6) (width 0.2) (layer "F.Cu") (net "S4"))
 (arc (start 142.707603 141.4) (mid 142.919735 141.487868) (end 143.007603 141.7) (width 0.2) (layer "F.Cu") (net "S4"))
 (segment (start 151.378346 131.027284) (end 151.40563 131.027284) (width 0.25) (layer "F.Cu") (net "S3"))
 (segment (start 148.891988 132.486358) (end 148.891988 132) (width 0.25) (layer "F.Cu") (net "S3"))
 (segment (start 149.891988 131.513642) (end 149.891988 132) (width 0.25) (layer "F.Cu") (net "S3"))
 (segment (start 152.891988 132.486358) (end 152.891988 132) (width 0.25) (layer "F.Cu") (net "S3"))
 (segment (start 146.891988 132) (end 146.891988 131.513642) (width 0.25) (layer "F.Cu") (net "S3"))
 (segment (start 146.36035 132.968362) (end 146.407807 132.968362) (width 0.25) (layer "F.Cu") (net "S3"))
 (segment (start 156.391988 132) (end 158.215131 132) (width 0.25) (layer "F.Cu") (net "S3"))
 (segment (start 149.378346 131.027284) (end 149.40563 131.027284) (width 0.25) (layer "F.Cu") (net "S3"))
 (segment (start 150.378346 132.972716) (end 150.40563 132.972716) (width 0.25) (layer "F.Cu") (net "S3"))
 (segment (start 127.414214 136) (end 138 136) (width 0.25) (layer "F.Cu") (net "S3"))
 (segment (start 106 133) (end 123.585786 133) (width 0.25) (layer "F.Cu") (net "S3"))
 (segment (start 151.891988 131.513642) (end 151.891988 132) (width 0.25) (layer "F.Cu") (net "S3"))
 (segment (start 154.891988 132) (end 154.891988 131.515829) (width 0.25) (layer "F.Cu") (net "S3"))
 (segment (start 124.292893 133.292893) (end 126.707107 135.707107) (width 0.25) (layer "F.Cu") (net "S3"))
 (segment (start 146.891988 132.484181) (end 146.891988 132) (width 0.25) (layer "F.Cu") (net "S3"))
 (segment (start 154.378346 132.972716) (end 154.40563 132.972716) (width 0.25) (layer "F.Cu") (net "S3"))
 (segment (start 151.891988 132) (end 151.891988 132.486358) (width 0.25) (layer "F.Cu") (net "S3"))
 (segment (start 150.891988 132) (end 150.891988 131.513642) (width 0.25) (layer "F.Cu") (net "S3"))
 (segment (start 155.376159 131.031658) (end 155.407817 131.031658) (width 0.25) (layer "F.Cu") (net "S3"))
 (segment (start 152.378346 132.972716) (end 152.40563 132.972716) (width 0.25) (layer "F.Cu") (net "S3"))
 (segment (start 148.891988 132) (end 148.891988 131.513642) (width 0.25) (layer "F.Cu") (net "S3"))
 (segment (start 147.891988 132) (end 147.891988 132.486358) (width 0.25) (layer "F.Cu") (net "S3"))
 (segment (start 158.215131 132) (end 164 132) (width 0.25) (layer "F.Cu") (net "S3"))
 (segment (start 153.891988 131.513642) (end 153.891988 132) (width 0.25) (layer "F.Cu") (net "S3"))
 (segment (start 150.891988 132.486358) (end 150.891988 132) (width 0.25) (layer "F.Cu") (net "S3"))
 (segment (start 153.891988 132) (end 153.891988 132.486358) (width 0.25) (layer "F.Cu") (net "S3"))
 (segment (start 147.891988 131.513642) (end 147.891988 132) (width 0.25) (layer "F.Cu") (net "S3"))
 (segment (start 147.378346 131.027284) (end 147.40563 131.027284) (width 0.25) (layer "F.Cu") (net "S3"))
 (segment (start 142 132) (end 145.391988 132) (width 0.25) (layer "F.Cu") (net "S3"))
 (segment (start 138 136) (end 142 132) (width 0.25) (layer "F.Cu") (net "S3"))
 (segment (start 153.378346 131.027284) (end 153.40563 131.027284) (width 0.25) (layer "F.Cu") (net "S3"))
 (segment (start 154.891988 132.486358) (end 154.891988 132) (width 0.25) (layer "F.Cu") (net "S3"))
 (segment (start 156.376159 132) (end 156.391988 132) (width 0.25) (layer "F.Cu") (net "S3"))
 (segment (start 148.378346 132.972716) (end 148.40563 132.972716) (width 0.25) (layer "F.Cu") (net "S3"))
 (segment (start 149.891988 132) (end 149.891988 132.486358) (width 0.25) (layer "F.Cu") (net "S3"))
 (segment (start 152.891988 132) (end 152.891988 131.513642) (width 0.25) (layer "F.Cu") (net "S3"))
 (arc (start 154.40563 132.972716) (mid 154.749537 132.830265) (end 154.891988 132.486358) (width 0.25) (layer "F.Cu") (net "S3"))
 (arc (start 152.891988 131.513642) (mid 153.034439 131.169735) (end 153.378346 131.027284) (width 0.25) (layer "F.Cu") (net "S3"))
 (arc (start 146.407807 132.968362) (mid 146.750175 132.826549) (end 146.891988 132.484181) (width 0.25) (layer "F.Cu") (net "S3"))
 (arc (start 150.40563 132.972716) (mid 150.749537 132.830265) (end 150.891988 132.486358) (width 0.25) (layer "F.Cu") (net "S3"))
 (arc (start 152.40563 132.972716) (mid 152.749537 132.830265) (end 152.891988 132.486358) (width 0.25) (layer "F.Cu") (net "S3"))
 (arc (start 147.40563 131.027284) (mid 147.749537 131.169735) (end 147.891988 131.513642) (width 0.25) (layer "F.Cu") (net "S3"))
 (arc (start 149.40563 131.027284) (mid 149.749537 131.169735) (end 149.891988 131.513642) (width 0.25) (layer "F.Cu") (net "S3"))
 (arc (start 155.891988 131.515829) (mid 156.033798 131.85819) (end 156.376159 132) (width 0.25) (layer "F.Cu") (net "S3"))
 (arc (start 151.891988 132.486358) (mid 152.034439 132.830265) (end 152.378346 132.972716) (width 0.25) (layer "F.Cu") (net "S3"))
 (arc (start 146.891988 131.513642) (mid 147.034439 131.169735) (end 147.378346 131.027284) (width 0.25) (layer "F.Cu") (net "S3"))
 (arc (start 145.876169 132.484181) (mid 146.017982 132.826549) (end 146.36035 132.968362) (width 0.25) (layer "F.Cu") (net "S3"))
 (arc (start 150.891988 131.513642) (mid 151.034439 131.169735) (end 151.378346 131.027284) (width 0.25) (layer "F.Cu") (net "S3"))
 (arc (start 153.891988 132.486358) (mid 154.034439 132.830265) (end 154.378346 132.972716) (width 0.25) (layer "F.Cu") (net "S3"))
 (arc (start 154.891988 131.515829) (mid 155.033798 131.173468) (end 155.376159 131.031658) (width 0.25) (layer "F.Cu") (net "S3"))
 (arc (start 126.707107 135.707107) (mid 127.03153 135.92388) (end 127.414214 136) (width 0.25) (layer "F.Cu") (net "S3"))
 (arc (start 153.40563 131.027284) (mid 153.749537 131.169735) (end 153.891988 131.513642) (width 0.25) (layer "F.Cu") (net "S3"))
 (arc (start 123.585786 133) (mid 123.96847 133.07612) (end 124.292893 133.292893) (width 0.25) (layer "F.Cu") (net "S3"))
 (arc (start 148.891988 131.513642) (mid 149.034439 131.169735) (end 149.378346 131.027284) (width 0.25) (layer "F.Cu") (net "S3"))
 (arc (start 148.40563 132.972716) (mid 148.749537 132.830265) (end 148.891988 132.486358) (width 0.25) (layer "F.Cu") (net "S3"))
 (arc (start 151.40563 131.027284) (mid 151.749537 131.169735) (end 151.891988 131.513642) (width 0.25) (layer "F.Cu") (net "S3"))
 (arc (start 149.891988 132.486358) (mid 150.034439 132.830265) (end 150.378346 132.972716) (width 0.25) (layer "F.Cu") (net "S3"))
 (arc (start 145.391988 132) (mid 145.734356 132.141813) (end 145.876169 132.484181) (width 0.25) (layer "F.Cu") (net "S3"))
 (arc (start 147.891988 132.486358) (mid 148.034439 132.830265) (end 148.378346 132.972716) (width 0.25) (layer "F.Cu") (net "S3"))
 (arc (start 155.407817 131.031658) (mid 155.750178 131.173468) (end 155.891988 131.515829) (width 0.25) (layer "F.Cu") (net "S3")))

